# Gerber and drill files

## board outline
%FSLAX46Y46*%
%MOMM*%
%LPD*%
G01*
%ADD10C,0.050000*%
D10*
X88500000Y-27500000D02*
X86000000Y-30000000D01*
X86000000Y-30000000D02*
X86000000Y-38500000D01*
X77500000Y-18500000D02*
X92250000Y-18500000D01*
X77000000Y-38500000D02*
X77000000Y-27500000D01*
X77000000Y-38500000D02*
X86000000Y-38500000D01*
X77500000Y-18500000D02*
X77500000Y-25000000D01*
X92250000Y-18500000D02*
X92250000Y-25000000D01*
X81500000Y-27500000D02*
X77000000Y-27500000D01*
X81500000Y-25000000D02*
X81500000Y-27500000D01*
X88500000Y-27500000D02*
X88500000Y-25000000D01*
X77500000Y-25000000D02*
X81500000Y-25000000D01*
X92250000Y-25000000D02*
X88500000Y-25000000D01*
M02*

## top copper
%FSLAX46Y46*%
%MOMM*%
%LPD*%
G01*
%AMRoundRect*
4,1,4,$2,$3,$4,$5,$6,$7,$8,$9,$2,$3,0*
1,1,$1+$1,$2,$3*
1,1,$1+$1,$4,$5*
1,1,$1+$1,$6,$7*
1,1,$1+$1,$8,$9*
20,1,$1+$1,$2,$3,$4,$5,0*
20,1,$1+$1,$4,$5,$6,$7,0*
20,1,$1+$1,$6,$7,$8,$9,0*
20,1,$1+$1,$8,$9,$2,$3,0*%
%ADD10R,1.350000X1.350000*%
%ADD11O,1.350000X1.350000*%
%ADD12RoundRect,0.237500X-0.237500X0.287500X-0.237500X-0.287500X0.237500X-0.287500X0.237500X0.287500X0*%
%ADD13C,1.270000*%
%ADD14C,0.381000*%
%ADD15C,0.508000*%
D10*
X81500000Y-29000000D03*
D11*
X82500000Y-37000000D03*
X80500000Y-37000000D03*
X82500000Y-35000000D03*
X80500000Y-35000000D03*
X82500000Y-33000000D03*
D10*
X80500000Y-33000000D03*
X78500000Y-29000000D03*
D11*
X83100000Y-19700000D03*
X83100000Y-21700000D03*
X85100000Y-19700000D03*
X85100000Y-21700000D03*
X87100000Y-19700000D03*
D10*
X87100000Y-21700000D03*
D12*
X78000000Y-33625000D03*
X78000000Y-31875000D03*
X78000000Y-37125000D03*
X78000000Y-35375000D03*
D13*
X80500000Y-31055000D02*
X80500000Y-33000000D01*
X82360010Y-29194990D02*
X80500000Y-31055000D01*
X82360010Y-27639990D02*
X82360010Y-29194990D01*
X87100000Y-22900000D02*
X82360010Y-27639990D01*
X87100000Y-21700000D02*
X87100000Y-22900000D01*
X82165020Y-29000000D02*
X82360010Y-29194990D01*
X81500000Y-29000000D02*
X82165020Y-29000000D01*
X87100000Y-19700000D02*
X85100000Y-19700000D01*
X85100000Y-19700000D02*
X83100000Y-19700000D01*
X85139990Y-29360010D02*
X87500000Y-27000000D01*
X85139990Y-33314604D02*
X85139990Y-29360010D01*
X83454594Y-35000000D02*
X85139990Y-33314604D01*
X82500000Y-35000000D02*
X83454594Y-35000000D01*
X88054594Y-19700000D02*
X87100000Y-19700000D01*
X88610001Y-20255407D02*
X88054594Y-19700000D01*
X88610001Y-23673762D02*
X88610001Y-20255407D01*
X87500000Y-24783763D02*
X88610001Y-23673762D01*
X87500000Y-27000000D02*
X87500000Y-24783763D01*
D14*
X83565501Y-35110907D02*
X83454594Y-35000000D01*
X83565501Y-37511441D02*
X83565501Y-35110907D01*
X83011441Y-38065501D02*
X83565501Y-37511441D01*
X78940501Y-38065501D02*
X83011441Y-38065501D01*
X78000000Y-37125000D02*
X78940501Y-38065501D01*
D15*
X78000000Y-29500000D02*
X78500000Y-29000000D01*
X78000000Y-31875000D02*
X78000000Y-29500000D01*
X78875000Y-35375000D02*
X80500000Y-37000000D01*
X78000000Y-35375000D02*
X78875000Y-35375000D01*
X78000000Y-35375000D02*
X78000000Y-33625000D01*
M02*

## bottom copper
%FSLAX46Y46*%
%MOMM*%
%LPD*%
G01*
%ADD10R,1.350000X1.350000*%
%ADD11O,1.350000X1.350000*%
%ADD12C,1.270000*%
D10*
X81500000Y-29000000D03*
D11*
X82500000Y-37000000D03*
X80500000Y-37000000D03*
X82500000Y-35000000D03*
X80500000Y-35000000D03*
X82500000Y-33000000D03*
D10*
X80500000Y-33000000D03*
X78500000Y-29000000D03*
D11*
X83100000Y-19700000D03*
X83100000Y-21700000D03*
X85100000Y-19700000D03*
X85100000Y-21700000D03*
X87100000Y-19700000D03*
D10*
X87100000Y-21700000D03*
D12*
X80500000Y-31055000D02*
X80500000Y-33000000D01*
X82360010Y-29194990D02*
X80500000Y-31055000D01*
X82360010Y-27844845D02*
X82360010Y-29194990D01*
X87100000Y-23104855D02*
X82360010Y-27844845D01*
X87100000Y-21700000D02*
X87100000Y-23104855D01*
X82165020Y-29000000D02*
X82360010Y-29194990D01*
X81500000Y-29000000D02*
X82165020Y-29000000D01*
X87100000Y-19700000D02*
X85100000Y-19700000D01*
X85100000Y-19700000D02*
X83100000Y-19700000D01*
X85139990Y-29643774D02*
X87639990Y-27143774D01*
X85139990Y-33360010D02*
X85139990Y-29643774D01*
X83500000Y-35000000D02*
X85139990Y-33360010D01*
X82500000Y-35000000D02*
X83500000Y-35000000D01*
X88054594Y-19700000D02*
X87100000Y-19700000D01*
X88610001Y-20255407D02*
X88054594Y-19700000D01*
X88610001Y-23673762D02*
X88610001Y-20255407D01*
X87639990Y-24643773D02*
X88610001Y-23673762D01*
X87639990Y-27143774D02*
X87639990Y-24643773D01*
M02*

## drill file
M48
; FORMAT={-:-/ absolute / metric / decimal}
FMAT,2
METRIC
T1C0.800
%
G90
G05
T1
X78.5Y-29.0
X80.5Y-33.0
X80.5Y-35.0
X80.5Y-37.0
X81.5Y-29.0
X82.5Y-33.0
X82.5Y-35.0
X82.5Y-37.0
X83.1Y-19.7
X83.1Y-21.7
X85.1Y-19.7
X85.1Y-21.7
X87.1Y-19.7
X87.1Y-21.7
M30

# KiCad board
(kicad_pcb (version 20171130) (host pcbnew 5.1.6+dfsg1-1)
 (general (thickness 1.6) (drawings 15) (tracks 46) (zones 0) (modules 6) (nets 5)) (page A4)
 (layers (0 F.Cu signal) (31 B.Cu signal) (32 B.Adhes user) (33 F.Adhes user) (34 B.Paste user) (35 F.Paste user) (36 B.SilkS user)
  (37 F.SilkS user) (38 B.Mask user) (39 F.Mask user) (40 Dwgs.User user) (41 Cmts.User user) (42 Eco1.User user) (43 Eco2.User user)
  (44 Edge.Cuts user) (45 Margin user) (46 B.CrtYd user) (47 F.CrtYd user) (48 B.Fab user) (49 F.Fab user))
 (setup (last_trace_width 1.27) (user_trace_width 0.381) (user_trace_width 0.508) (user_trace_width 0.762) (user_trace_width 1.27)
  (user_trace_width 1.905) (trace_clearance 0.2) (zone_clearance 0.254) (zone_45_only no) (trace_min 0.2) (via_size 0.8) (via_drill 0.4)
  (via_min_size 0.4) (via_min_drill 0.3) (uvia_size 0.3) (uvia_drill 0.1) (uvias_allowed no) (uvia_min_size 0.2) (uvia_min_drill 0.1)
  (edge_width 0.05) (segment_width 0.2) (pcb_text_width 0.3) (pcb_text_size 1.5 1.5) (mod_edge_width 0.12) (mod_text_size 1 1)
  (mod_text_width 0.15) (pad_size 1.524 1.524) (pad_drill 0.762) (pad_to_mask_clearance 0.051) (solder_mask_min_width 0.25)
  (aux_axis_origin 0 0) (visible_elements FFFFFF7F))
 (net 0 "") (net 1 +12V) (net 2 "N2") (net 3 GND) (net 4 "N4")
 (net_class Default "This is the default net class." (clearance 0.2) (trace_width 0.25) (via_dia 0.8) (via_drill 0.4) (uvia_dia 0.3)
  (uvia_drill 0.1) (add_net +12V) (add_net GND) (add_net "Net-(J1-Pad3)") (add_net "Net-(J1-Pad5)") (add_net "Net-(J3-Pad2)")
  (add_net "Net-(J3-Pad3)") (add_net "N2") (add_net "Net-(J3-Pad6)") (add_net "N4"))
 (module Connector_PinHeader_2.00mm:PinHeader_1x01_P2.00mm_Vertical (layer F.Cu) (at 81.5 29)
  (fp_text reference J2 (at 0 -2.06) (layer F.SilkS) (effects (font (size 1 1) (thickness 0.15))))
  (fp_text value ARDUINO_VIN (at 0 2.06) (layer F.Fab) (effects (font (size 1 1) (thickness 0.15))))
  (pad 1 thru_hole rect (at 0 0) (size 1.35 1.35) (drill 0.8) (layers *.Cu *.Mask) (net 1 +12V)))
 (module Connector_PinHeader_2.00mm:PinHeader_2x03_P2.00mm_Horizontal (layer F.Cu) (at 80.5 33)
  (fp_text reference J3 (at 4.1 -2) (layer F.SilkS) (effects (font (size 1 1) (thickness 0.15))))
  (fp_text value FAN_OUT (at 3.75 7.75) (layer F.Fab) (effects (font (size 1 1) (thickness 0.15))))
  (pad 6 thru_hole oval (at 2 4) (size 1.35 1.35) (drill 0.8) (layers *.Cu *.Mask))
  (pad 5 thru_hole oval (at 0 4) (size 1.35 1.35) (drill 0.8) (layers *.Cu *.Mask) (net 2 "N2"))
  (pad 4 thru_hole oval (at 2 2) (size 1.35 1.35) (drill 0.8) (layers *.Cu *.Mask) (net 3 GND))
  (pad 3 thru_hole oval (at 0 2) (size 1.35 1.35) (drill 0.8) (layers *.Cu *.Mask))
  (pad 2 thru_hole oval (at 2 0) (size 1.35 1.35) (drill 0.8) (layers *.Cu *.Mask))
  (pad 1 thru_hole rect (at 0 0) (size 1.35 1.35) (drill 0.8) (layers *.Cu *.Mask) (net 1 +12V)))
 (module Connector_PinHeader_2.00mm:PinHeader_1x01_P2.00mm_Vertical (layer F.Cu) (at 78.5 29)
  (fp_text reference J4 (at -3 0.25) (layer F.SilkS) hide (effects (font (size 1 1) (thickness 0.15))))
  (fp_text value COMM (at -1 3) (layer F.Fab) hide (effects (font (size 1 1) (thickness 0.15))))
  (pad 1 thru_hole rect (at 0 0) (size 1.35 1.35) (drill 0.8) (layers *.Cu *.Mask) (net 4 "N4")))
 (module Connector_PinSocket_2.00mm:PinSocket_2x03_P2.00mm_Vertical (layer F.Cu) (at 87.1 21.7 270)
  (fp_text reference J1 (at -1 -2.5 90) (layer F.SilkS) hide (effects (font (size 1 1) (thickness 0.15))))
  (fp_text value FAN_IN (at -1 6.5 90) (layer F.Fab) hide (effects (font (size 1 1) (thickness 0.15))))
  (pad 6 thru_hole oval (at -2 4 270) (size 1.35 1.35) (drill 0.8) (layers *.Cu *.Mask) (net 3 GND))
  (pad 5 thru_hole oval (at 0 4 270) (size 1.35 1.35) (drill 0.8) (layers *.Cu *.Mask))
  (pad 4 thru_hole oval (at -2 2 270) (size 1.35 1.35) (drill 0.8) (layers *.Cu *.Mask) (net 3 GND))
  (pad 3 thru_hole oval (at 0 2 270) (size 1.35 1.35) (drill 0.8) (layers *.Cu *.Mask))
  (pad 2 thru_hole oval (at -2 0 270) (size 1.35 1.35) (drill 0.8) (layers *.Cu *.Mask) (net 3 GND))
  (pad 1 thru_hole rect (at 0 0 270) (size 1.35 1.35) (drill 0.8) (layers *.Cu *.Mask) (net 1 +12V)))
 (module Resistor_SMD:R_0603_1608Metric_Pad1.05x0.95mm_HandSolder (layer F.Cu) (at 78 32.75 270)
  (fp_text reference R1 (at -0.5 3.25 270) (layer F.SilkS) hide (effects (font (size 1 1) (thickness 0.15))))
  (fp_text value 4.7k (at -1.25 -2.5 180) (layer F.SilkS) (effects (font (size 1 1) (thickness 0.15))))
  (pad 2 smd roundrect (at 0.875 0 270) (size 1.05 0.95) (layers F.Cu F.Paste F.Mask) (roundrect_rratio 0.25) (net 2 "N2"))
  (pad 1 smd roundrect (at -0.875 0 270) (size 1.05 0.95) (layers F.Cu F.Paste F.Mask) (roundrect_rratio 0.25) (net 4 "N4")))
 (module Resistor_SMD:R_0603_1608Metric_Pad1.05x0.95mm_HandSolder (layer F.Cu) (at 78 36.25 270)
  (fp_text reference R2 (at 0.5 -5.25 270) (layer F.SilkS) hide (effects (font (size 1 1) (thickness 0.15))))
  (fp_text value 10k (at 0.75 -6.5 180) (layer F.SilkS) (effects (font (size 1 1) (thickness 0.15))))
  (pad 2 smd roundrect (at 0.875 0 270) (size 1.05 0.95) (layers F.Cu F.Paste F.Mask) (roundrect_rratio 0.25) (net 3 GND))
  (pad 1 smd roundrect (at -0.875 0 270) (size 1.05 0.95) (layers F.Cu F.Paste F.Mask) (roundrect_rratio 0.25) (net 2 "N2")))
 (gr_line (start 88.5 27.5) (end 86 30) (layer Edge.Cuts) (width 0.05))
 (gr_line (start 86 30) (end 86 38.5) (layer Edge.Cuts) (width 0.05))
 (gr_line (start 77.5 18.5) (end 92.25 18.5) (layer Edge.Cuts) (width 0.05))
 (gr_line (start 77 38.5) (end 77 27.5) (layer Edge.Cuts) (width 0.05))
 (gr_line (start 77 38.5) (end 86 38.5) (layer Edge.Cuts) (width 0.05))
 (gr_line (start 77.5 18.5) (end 77.5 25) (layer Edge.Cuts) (width 0.05))
 (gr_line (start 92.25 18.5) (end 92.25 25) (layer Edge.Cuts) (width 0.05))
 (gr_line (start 81.5 27.5) (end 77 27.5) (layer Edge.Cuts) (width 0.05))
 (gr_line (start 81.5 25) (end 81.5 27.5) (layer Edge.Cuts) (width 0.05))
 (gr_line (start 88.5 27.5) (end 88.5 25) (layer Edge.Cuts) (width 0.05))
 (gr_line (start 77.5 25) (end 81.5 25) (layer Edge.Cuts) (width 0.05))
 (gr_line (start 92.25 25) (end 88.5 25) (layer Edge.Cuts) (width 0.05))
 (segment (start 80.5 31.055) (end 80.5 33) (width 1.27) (layer F.Cu) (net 1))
 (segment (start 82.36001 29.19499) (end 80.5 31.055) (width 1.27) (layer F.Cu) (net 1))
 (segment (start 82.36001 27.63999) (end 82.36001 29.19499) (width 1.27) (layer F.Cu) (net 1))
 (segment (start 87.1 22.9) (end 82.36001 27.63999) (width 1.27) (layer F.Cu) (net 1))
 (segment (start 87.1 21.7) (end 87.1 22.9) (width 1.27) (layer F.Cu) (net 1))
 (segment (start 80.5 31.055) (end 80.5 33) (width 1.27) (layer B.Cu) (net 1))
 (segment (start 82.36001 29.19499) (end 80.5 31.055) (width 1.27) (layer B.Cu) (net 1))
 (segment (start 82.36001 27.844845) (end 82.36001 29.19499) (width 1.27) (layer B.Cu) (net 1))
 (segment (start 87.1 23.104855) (end 82.36001 27.844845) (width 1.27) (layer B.Cu) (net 1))
 (segment (start 87.1 21.7) (end 87.1 23.104855) (width 1.27) (layer B.Cu) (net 1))
 (segment (start 82.16502 29) (end 82.36001 29.19499) (width 1.27) (layer F.Cu) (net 1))
 (segment (start 81.5 29) (end 82.16502 29) (width 1.27) (layer F.Cu) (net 1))
 (segment (start 82.16502 29) (end 82.36001 29.19499) (width 1.27) (layer B.Cu) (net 1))
 (segment (start 81.5 29) (end 82.16502 29) (width 1.27) (layer B.Cu) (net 1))
 (segment (start 87.1 19.7) (end 85.1 19.7) (width 1.27) (layer F.Cu) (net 3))
 (segment (start 85.1 19.7) (end 83.1 19.7) (width 1.27) (layer F.Cu) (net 3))
 (segment (start 87.1 19.7) (end 85.1 19.7) (width 1.27) (layer B.Cu) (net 3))
 (segment (start 85.1 19.7) (end 83.1 19.7) (width 1.27) (layer B.Cu) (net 3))
 (segment (start 85.13999 29.36001) (end 87.5 27) (width 1.27) (layer F.Cu) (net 3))
 (segment (start 85.13999 33.314604) (end 85.13999 29.36001) (width 1.27) (layer F.Cu) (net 3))
 (segment (start 83.454594 35) (end 85.13999 33.314604) (width 1.27) (layer F.Cu) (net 3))
 (segment (start 82.5 35) (end 83.454594 35) (width 1.27) (layer F.Cu) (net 3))
 (segment (start 88.054594 19.7) (end 87.1 19.7) (width 1.27) (layer F.Cu) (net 3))
 (segment (start 88.610001 20.255407) (end 88.054594 19.7) (width 1.27) (layer F.Cu) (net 3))
 (segment (start 88.610001 23.673762) (end 88.610001 20.255407) (width 1.27) (layer F.Cu) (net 3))
 (segment (start 87.5 24.783763) (end 88.610001 23.673762) (width 1.27) (layer F.Cu) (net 3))
 (segment (start 87.5 27) (end 87.5 24.783763) (width 1.27) (layer F.Cu) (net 3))
 (segment (start 85.13999 29.643774) (end 87.63999 27.143774) (width 1.27) (layer B.Cu) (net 3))
 (segment (start 85.13999 33.36001) (end 85.13999 29.643774) (width 1.27) (layer B.Cu) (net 3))
 (segment (start 83.5 35) (end 85.13999 33.36001) (width 1.27) (layer B.Cu) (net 3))
 (segment (start 82.5 35) (end 83.5 35) (width 1.27) (layer B.Cu) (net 3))
 (segment (start 88.054594 19.7) (end 87.1 19.7) (width 1.27) (layer B.Cu) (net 3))
 (segment (start 88.610001 20.255407) (end 88.054594 19.7) (width 1.27) (layer B.Cu) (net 3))
 (segment (start 88.610001 23.673762) (end 88.610001 20.255407) (width 1.27) (layer B.Cu) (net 3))
 (segment (start 87.63999 24.643773) (end 88.610001 23.673762) (width 1.27) (layer B.Cu) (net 3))
 (segment (start 87.63999 27.143774) (end 87.63999 24.643773) (width 1.27) (layer B.Cu) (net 3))
 (segment (start 83.565501 35.110907) (end 83.454594 35) (width 0.381) (layer F.Cu) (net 3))
 (segment (start 83.565501 37.511441) (end 83.565501 35.110907) (width 0.381) (layer F.Cu) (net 3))
 (segment (start 83.011441 38.065501) (end 83.565501 37.511441) (width 0.381) (layer F.Cu) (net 3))
 (segment (start 78.940501 38.065501) (end 83.011441 38.065501) (width 0.381) (layer F.Cu) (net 3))
 (segment (start 78 37.125) (end 78.940501 38.065501) (width 0.381) (layer F.Cu) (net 3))
 (segment (start 78 29.5) (end 78.5 29) (width 0.508) (layer F.Cu) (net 4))
 (segment (start 78 31.875) (end 78 29.5) (width 0.508) (layer F.Cu) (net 4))
 (segment (start 78.875 35.375) (end 80.5 37) (width 0.508) (layer F.Cu) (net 2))
 (segment (start 78 35.375) (end 78.875 35.375) (width 0.508) (layer F.Cu) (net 2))
 (segment (start 78 35.375) (end 78 33.625) (width 0.508) (layer F.Cu) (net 2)))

